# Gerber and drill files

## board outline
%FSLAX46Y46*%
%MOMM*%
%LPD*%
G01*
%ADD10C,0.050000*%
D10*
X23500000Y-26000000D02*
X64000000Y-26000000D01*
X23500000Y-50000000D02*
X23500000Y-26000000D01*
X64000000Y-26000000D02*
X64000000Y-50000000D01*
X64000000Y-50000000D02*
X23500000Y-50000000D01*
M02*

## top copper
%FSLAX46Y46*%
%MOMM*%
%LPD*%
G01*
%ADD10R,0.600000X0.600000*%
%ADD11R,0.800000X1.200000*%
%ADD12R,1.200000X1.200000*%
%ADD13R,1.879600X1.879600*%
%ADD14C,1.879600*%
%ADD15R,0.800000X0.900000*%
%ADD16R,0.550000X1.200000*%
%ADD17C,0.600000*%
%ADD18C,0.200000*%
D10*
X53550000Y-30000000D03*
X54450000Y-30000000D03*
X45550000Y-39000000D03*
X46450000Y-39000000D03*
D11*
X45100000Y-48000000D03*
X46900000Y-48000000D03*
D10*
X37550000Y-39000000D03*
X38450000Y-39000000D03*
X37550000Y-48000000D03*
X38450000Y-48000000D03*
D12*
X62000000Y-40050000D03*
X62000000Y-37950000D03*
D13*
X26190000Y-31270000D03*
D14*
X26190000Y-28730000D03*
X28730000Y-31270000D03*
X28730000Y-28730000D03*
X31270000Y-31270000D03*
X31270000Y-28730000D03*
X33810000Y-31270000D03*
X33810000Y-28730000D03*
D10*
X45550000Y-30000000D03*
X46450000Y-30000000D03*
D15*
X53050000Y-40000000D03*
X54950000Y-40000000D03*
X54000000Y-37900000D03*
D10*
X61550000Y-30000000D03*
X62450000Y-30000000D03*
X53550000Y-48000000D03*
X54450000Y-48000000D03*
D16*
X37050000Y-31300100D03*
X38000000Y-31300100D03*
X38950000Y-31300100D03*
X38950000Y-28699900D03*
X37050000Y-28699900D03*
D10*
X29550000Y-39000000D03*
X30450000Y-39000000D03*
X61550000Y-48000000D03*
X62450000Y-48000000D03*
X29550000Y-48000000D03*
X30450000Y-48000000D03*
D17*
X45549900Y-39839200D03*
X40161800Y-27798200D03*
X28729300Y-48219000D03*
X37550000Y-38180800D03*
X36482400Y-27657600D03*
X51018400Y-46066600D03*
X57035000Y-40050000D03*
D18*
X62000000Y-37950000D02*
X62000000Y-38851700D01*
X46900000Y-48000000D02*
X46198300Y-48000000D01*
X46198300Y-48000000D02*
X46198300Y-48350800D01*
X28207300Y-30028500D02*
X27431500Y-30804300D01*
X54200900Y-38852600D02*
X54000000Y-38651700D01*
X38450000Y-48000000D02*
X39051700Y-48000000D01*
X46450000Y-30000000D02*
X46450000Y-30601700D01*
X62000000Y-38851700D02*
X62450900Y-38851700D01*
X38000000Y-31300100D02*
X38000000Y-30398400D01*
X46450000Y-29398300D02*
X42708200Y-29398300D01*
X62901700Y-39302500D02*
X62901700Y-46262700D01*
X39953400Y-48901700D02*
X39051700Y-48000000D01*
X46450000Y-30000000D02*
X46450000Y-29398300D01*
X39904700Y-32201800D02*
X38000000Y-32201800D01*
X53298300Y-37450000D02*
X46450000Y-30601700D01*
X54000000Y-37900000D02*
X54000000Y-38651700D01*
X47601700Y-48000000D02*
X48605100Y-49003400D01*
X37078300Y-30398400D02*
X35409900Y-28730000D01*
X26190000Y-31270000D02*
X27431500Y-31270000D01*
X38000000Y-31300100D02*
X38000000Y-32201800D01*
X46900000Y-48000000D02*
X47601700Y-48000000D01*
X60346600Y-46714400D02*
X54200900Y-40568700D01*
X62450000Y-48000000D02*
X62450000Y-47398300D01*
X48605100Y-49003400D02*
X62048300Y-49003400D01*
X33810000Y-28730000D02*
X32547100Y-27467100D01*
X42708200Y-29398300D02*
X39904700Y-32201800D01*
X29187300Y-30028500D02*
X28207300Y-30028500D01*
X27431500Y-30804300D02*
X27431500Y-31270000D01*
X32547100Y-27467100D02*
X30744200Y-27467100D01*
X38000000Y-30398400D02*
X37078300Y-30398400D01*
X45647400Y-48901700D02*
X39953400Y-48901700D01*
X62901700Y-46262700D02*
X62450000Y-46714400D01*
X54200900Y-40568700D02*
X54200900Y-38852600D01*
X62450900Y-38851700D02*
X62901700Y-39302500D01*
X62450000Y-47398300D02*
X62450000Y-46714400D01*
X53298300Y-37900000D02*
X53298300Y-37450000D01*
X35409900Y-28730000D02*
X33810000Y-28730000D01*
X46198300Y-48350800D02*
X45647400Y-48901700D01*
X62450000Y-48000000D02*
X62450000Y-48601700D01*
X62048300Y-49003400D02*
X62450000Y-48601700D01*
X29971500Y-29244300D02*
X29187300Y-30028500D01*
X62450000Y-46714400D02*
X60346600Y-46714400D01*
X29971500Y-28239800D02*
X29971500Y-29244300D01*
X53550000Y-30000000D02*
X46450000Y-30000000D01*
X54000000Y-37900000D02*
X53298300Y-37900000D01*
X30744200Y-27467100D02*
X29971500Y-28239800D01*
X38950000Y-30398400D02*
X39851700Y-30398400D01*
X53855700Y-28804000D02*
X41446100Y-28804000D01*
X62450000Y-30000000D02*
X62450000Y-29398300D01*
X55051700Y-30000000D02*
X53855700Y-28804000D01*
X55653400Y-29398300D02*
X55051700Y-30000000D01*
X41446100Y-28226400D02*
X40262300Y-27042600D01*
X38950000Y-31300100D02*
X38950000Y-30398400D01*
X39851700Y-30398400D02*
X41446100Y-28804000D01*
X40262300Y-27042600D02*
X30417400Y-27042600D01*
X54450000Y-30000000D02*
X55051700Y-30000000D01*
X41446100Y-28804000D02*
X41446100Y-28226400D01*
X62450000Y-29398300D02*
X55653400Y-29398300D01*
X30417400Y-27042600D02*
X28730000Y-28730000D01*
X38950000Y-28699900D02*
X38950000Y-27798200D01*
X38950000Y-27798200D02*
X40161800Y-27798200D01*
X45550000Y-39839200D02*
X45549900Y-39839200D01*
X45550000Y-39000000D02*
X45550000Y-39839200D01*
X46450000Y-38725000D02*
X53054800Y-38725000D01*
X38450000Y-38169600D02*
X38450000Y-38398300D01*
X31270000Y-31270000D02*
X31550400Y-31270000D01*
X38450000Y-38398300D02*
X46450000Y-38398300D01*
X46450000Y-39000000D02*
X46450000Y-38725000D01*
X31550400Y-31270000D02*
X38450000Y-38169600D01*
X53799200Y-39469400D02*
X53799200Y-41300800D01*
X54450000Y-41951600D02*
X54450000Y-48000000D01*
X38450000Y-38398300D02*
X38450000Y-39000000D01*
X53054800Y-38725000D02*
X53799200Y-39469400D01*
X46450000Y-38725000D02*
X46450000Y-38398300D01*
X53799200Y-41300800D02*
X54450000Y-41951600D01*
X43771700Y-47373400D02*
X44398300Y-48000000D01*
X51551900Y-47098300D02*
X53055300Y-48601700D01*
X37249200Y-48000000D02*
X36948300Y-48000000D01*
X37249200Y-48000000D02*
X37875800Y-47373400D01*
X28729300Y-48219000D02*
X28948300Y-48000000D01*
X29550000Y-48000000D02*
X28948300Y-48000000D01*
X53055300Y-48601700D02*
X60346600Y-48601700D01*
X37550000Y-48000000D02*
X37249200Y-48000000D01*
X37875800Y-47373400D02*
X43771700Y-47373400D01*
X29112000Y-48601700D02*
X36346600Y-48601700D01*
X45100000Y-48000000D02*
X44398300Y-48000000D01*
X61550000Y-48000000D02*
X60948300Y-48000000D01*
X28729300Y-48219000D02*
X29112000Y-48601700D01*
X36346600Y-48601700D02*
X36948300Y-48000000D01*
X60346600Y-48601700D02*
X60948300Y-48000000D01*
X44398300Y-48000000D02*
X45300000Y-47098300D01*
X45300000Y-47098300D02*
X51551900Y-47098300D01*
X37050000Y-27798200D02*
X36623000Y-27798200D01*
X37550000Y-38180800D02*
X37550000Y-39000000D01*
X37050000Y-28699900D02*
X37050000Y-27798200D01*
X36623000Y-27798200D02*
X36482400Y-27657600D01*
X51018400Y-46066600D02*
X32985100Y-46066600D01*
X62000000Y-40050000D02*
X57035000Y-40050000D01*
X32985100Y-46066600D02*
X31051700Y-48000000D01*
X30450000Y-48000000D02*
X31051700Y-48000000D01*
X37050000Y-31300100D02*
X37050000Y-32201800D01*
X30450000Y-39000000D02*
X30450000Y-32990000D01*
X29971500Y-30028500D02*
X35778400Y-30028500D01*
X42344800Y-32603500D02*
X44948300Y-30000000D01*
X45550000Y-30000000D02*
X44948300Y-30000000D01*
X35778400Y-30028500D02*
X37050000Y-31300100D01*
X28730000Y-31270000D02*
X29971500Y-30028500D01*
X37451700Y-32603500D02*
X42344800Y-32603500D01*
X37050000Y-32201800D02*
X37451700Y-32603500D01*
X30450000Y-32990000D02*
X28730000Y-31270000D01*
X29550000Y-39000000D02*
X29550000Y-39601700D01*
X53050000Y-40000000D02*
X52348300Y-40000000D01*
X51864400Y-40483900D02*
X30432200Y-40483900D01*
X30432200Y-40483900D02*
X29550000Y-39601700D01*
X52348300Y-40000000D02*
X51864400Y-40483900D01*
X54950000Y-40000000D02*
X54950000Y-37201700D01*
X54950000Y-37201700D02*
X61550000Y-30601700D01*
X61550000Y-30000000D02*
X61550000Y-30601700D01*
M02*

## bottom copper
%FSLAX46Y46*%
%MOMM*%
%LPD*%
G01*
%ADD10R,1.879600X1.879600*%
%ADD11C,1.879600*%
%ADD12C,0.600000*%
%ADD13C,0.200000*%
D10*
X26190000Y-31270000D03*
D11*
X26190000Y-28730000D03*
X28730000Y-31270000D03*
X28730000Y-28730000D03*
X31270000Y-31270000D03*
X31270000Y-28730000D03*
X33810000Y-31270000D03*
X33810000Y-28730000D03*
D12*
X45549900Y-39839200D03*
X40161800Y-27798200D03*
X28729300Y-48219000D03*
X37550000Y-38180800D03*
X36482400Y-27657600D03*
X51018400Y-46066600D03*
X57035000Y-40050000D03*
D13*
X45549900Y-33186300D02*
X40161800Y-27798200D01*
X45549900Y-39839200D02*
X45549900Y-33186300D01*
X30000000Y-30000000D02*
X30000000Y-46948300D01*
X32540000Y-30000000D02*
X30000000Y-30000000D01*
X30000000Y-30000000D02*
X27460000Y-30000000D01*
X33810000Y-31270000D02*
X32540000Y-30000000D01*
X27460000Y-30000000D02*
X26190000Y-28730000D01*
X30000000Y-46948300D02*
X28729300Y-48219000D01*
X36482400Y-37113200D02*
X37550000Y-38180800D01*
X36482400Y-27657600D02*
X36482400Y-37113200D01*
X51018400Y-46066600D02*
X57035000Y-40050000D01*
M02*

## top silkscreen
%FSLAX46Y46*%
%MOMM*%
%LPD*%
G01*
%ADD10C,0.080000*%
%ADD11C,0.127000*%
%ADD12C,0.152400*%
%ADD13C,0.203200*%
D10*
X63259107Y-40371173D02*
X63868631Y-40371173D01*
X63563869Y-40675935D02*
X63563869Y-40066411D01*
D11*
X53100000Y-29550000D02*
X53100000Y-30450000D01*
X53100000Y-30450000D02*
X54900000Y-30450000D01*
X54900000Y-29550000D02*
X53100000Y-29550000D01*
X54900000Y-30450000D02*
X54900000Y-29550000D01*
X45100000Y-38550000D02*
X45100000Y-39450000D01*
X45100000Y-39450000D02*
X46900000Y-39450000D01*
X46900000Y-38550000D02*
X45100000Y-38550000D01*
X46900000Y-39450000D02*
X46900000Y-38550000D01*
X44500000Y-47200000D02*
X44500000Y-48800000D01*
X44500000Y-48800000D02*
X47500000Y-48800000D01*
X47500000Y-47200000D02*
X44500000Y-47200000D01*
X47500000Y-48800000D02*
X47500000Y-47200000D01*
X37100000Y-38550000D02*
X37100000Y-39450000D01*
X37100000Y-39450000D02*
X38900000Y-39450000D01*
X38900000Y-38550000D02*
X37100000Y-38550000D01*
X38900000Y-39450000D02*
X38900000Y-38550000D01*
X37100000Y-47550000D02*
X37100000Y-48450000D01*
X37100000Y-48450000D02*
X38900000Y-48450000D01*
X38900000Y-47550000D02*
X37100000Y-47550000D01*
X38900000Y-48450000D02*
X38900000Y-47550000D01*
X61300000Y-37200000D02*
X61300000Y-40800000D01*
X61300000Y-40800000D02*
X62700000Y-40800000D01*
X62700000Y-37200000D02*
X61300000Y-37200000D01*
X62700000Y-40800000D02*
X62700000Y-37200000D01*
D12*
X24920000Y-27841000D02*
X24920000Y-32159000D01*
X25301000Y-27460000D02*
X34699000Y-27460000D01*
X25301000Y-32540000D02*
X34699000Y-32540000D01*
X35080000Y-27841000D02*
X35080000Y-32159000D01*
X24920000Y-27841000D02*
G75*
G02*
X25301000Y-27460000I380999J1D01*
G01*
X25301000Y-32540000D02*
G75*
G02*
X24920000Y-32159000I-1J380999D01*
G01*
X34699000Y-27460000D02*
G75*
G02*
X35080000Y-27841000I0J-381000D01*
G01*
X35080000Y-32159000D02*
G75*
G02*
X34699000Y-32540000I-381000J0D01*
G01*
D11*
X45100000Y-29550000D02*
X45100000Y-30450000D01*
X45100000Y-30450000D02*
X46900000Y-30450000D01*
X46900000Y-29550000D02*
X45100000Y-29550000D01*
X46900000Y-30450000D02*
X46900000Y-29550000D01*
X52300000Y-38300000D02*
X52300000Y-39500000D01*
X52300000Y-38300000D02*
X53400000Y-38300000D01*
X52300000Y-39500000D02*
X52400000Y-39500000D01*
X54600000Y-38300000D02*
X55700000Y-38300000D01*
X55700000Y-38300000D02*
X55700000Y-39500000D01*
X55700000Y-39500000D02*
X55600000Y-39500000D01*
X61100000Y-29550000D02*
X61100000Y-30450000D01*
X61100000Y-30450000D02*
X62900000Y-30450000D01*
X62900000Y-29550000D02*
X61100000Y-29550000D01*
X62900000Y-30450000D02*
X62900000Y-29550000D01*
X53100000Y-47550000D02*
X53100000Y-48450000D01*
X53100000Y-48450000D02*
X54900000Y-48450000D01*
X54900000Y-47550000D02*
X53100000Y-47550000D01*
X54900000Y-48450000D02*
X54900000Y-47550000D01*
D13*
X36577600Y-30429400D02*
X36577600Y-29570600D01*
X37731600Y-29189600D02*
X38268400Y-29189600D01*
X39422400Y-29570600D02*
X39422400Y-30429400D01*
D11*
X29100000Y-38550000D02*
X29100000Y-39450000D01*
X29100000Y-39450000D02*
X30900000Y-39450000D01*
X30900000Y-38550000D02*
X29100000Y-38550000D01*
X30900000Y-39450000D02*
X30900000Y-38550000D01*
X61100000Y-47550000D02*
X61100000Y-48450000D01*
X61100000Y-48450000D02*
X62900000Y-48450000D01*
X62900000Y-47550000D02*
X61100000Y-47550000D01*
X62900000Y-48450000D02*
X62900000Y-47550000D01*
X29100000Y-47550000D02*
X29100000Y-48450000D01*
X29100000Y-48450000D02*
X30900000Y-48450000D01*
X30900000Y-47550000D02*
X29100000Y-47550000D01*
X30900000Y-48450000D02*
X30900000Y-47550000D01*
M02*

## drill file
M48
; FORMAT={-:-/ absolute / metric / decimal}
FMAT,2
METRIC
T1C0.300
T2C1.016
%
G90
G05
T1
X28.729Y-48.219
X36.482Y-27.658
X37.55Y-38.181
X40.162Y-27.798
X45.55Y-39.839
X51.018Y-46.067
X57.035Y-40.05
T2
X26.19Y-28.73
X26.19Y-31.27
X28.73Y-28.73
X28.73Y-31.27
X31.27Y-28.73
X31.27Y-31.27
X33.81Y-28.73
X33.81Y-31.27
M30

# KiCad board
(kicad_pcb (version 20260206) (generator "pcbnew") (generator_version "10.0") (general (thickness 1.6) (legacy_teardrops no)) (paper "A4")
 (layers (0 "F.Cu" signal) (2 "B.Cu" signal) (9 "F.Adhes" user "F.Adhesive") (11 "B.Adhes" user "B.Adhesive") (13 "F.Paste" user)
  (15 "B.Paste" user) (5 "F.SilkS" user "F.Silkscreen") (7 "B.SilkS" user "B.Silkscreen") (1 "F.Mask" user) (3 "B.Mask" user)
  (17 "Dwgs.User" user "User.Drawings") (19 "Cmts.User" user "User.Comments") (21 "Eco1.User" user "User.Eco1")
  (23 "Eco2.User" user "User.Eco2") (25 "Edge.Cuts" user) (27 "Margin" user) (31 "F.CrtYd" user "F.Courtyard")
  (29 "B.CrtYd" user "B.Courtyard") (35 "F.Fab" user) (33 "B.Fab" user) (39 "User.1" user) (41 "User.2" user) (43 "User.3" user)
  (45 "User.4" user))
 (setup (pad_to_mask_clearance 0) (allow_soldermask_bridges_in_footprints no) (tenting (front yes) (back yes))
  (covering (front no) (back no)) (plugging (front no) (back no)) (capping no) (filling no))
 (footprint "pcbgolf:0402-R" (layer "F.Cu") (at 54 30)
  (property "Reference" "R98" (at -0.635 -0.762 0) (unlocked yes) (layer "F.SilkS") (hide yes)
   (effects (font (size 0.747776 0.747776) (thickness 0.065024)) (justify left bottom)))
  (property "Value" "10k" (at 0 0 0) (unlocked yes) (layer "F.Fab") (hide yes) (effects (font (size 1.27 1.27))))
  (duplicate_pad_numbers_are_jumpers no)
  (fp_line (start -0.9 -0.45) (end -0.9 0.45) (stroke (width 0.127) (type solid)) (layer "F.SilkS"))
  (fp_line (start -0.9 0.45) (end 0.9 0.45) (stroke (width 0.127) (type solid)) (layer "F.SilkS"))
  (fp_line (start 0.9 -0.45) (end -0.9 -0.45) (stroke (width 0.127) (type solid)) (layer "F.SilkS"))
  (fp_line (start 0.9 0.45) (end 0.9 -0.45) (stroke (width 0.127) (type solid)) (layer "F.SilkS"))
  (pad "1" smd rect (at -0.45 0) (size 0.6 0.6) (layers "F.Cu" "F.Mask" "F.Paste") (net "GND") (solder_mask_margin 0.0508)
   (solder_paste_margin 0) (thermal_bridge_angle 0))
  (pad "2" smd rect (at 0.45 0) (size 0.6 0.6) (layers "F.Cu" "F.Mask" "F.Paste") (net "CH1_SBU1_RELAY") (solder_mask_margin 0.0508)
   (solder_paste_margin 0) (thermal_bridge_angle 0)))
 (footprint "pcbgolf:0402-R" (layer "F.Cu") (at 46 39)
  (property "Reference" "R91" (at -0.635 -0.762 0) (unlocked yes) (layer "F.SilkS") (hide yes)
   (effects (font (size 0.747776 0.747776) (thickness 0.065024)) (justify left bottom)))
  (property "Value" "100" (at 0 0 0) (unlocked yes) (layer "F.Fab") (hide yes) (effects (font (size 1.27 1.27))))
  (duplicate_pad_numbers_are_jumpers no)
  (fp_line (start -0.9 -0.45) (end -0.9 0.45) (stroke (width 0.127) (type solid)) (layer "F.SilkS"))
  (fp_line (start -0.9 0.45) (end 0.9 0.45) (stroke (width 0.127) (type solid)) (layer "F.SilkS"))
  (fp_line (start 0.9 -0.45) (end -0.9 -0.45) (stroke (width 0.127) (type solid)) (layer "F.SilkS"))
  (fp_line (start 0.9 0.45) (end 0.9 -0.45) (stroke (width 0.127) (type solid)) (layer "F.SilkS"))
  (pad "1" smd rect (at -0.45 0) (size 0.6 0.6) (layers "F.Cu" "F.Mask" "F.Paste") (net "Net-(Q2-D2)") (solder_mask_margin 0.0508)
   (solder_paste_margin 0) (thermal_bridge_angle 0))
  (pad "2" smd rect (at 0.45 0) (size 0.6 0.6) (layers "F.Cu" "F.Mask" "F.Paste") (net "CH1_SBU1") (solder_mask_margin 0.0508)
   (solder_paste_margin 0) (thermal_bridge_angle 0)))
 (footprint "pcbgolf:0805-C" (layer "F.Cu") (at 46 48)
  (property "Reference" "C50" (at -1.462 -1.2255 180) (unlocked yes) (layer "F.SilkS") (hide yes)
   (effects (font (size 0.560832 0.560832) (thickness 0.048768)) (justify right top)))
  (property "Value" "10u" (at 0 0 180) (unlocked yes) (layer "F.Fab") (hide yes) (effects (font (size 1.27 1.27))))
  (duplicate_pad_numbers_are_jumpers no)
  (fp_line (start -1.5 -0.8) (end -1.5 0.8) (stroke (width 0.127) (type solid)) (layer "F.SilkS"))
  (fp_line (start -1.5 0.8) (end 1.5 0.8) (stroke (width 0.127) (type solid)) (layer "F.SilkS"))
  (fp_line (start 1.5 -0.8) (end -1.5 -0.8) (stroke (width 0.127) (type solid)) (layer "F.SilkS"))
  (fp_line (start 1.5 0.8) (end 1.5 -0.8) (stroke (width 0.127) (type solid)) (layer "F.SilkS"))
  (pad "1" smd rect (at -0.9 0) (size 0.8 1.2) (layers "F.Cu" "F.Mask" "F.Paste") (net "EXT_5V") (solder_mask_margin 0.0508)
   (solder_paste_margin 0) (thermal_bridge_angle 0))
  (pad "2" smd rect (at 0.9 0) (size 0.8 1.2) (layers "F.Cu" "F.Mask" "F.Paste") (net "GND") (solder_mask_margin 0.0508)
   (solder_paste_margin 0) (thermal_bridge_angle 0)))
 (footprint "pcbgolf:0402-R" (layer "F.Cu") (at 38 39)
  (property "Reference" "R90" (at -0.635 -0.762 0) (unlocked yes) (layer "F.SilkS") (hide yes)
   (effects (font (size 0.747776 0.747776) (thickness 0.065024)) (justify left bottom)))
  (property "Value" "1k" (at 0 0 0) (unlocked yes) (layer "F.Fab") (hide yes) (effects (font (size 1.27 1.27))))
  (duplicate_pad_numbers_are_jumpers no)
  (fp_line (start -0.9 -0.45) (end -0.9 0.45) (stroke (width 0.127) (type solid)) (layer "F.SilkS"))
  (fp_line (start -0.9 0.45) (end 0.9 0.45) (stroke (width 0.127) (type solid)) (layer "F.SilkS"))
  (fp_line (start 0.9 -0.45) (end -0.9 -0.45) (stroke (width 0.127) (type solid)) (layer "F.SilkS"))
  (fp_line (start 0.9 0.45) (end 0.9 -0.45) (stroke (width 0.127) (type solid)) (layer "F.SilkS"))
  (pad "1" smd rect (at -0.45 0) (size 0.6 0.6) (layers "F.Cu" "F.Mask" "F.Paste") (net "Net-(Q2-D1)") (solder_mask_margin 0.0508)
   (solder_paste_margin 0) (thermal_bridge_angle 0))
  (pad "2" smd rect (at 0.45 0) (size 0.6 0.6) (layers "F.Cu" "F.Mask" "F.Paste") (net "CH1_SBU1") (solder_mask_margin 0.0508)
   (solder_paste_margin 0) (thermal_bridge_angle 0)))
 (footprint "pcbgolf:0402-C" (layer "F.Cu") (at 38 48)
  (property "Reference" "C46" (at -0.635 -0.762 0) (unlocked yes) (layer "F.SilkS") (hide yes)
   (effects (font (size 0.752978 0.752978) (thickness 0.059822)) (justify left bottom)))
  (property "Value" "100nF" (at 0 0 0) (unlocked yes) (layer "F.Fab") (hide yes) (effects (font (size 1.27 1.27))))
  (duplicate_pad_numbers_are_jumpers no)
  (fp_line (start -0.9 -0.45) (end -0.9 0.45) (stroke (width 0.127) (type solid)) (layer "F.SilkS"))
  (fp_line (start -0.9 0.45) (end 0.9 0.45) (stroke (width 0.127) (type solid)) (layer "F.SilkS"))
  (fp_line (start 0.9 -0.45) (end -0.9 -0.45) (stroke (width 0.127) (type solid)) (layer "F.SilkS"))
  (fp_line (start 0.9 0.45) (end 0.9 -0.45) (stroke (width 0.127) (type solid)) (layer "F.SilkS"))
  (pad "1" smd rect (at -0.45 0) (size 0.6 0.6) (layers "F.Cu" "F.Mask" "F.Paste") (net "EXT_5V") (solder_mask_margin 0.0508)
   (solder_paste_margin 0) (thermal_bridge_angle 0))
  (pad "2" smd rect (at 0.45 0) (size 0.6 0.6) (layers "F.Cu" "F.Mask" "F.Paste") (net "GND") (solder_mask_margin 0.0508)
   (solder_paste_margin 0) (thermal_bridge_angle 0)))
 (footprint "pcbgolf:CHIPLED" (layer "F.Cu") (at 62 39)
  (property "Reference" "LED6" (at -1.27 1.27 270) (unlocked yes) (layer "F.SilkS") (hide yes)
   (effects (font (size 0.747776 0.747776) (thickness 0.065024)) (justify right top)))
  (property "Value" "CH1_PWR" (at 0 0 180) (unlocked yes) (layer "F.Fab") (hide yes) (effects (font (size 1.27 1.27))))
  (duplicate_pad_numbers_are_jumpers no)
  (fp_line (start -0.7 -1.8) (end -0.7 1.8) (stroke (width 0.127) (type solid)) (layer "F.SilkS"))
  (fp_line (start -0.7 1.8) (end 0.7 1.8) (stroke (width 0.127) (type solid)) (layer "F.SilkS"))
  (fp_line (start 0.7 -1.8) (end -0.7 -1.8) (stroke (width 0.127) (type solid)) (layer "F.SilkS"))
  (fp_line (start 0.7 1.8) (end 0.7 -1.8) (stroke (width 0.127) (type solid)) (layer "F.SilkS"))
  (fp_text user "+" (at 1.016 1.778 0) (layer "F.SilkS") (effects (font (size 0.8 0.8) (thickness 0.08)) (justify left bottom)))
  (pad "A" smd rect (at 0 1.05) (size 1.2 1.2) (layers "F.Cu" "F.Mask" "F.Paste") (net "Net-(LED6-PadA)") (solder_mask_margin 0.0508)
   (solder_paste_margin 0) (thermal_bridge_angle 0))
  (pad "C" smd rect (at 0 -1.05) (size 1.2 1.2) (layers "F.Cu" "F.Mask" "F.Paste") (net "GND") (solder_mask_margin 0.0508)
   (solder_paste_margin 0) (thermal_bridge_angle 0)))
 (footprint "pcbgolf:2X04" (layer "F.Cu") (at 30 30)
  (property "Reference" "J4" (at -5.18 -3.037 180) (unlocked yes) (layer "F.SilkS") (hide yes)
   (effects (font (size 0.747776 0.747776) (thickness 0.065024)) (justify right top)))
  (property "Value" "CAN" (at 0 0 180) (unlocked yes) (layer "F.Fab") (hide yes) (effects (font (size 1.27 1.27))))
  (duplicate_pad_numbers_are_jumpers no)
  (fp_line (start -5.08 -2.159) (end -5.08 2.159) (stroke (width 0.1524) (type solid)) (layer "F.SilkS"))
  (fp_line (start -4.699 -2.54) (end 4.699 -2.54) (stroke (width 0.1524) (type solid)) (layer "F.SilkS"))
  (fp_line (start -4.699 2.54) (end 4.699 2.54) (stroke (width 0.1524) (type solid)) (layer "F.SilkS"))
  (fp_line (start 5.08 -2.159) (end 5.08 2.159) (stroke (width 0.1524) (type solid)) (layer "F.SilkS"))
  (fp_arc (start -5.08 -2.159) (mid -4.968408 -2.428408) (end -4.699 -2.54) (stroke (width 0.1524) (type solid)) (layer "F.SilkS"))
  (fp_arc (start -4.699 2.54) (mid -4.968408 2.428408) (end -5.08 2.159) (stroke (width 0.1524) (type solid)) (layer "F.SilkS"))
  (fp_arc (start 4.699 -2.54) (mid 4.968408 -2.428408) (end 5.08 -2.159) (stroke (width 0.1524) (type solid)) (layer "F.SilkS"))
  (fp_arc (start 5.08 2.159) (mid 4.968408 2.428408) (end 4.699 2.54) (stroke (width 0.1524) (type solid)) (layer "F.SilkS"))
  (pad "1" thru_hole rect (at -3.81 1.27 90) (size 1.8796 1.8796) (drill 1.016) (layers "*.Cu" "*.Mask") (remove_unused_layers no)
   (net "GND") (solder_mask_margin 0.0508) (thermal_bridge_angle 0))
  (pad "2" thru_hole circle (at -3.81 -1.27 90) (size 1.8796 1.8796) (drill 1.016) (layers "*.Cu" "*.Mask") (remove_unused_layers no)
   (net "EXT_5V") (solder_mask_margin 0.0508) (thermal_bridge_angle 0))
  (pad "3" thru_hole circle (at -1.27 1.27 90) (size 1.8796 1.8796) (drill 1.016) (layers "*.Cu" "*.Mask") (remove_unused_layers no)
   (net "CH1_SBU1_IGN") (solder_mask_margin 0.0508) (thermal_bridge_angle 0))
  (pad "4" thru_hole circle (at -1.27 -1.27 90) (size 1.8796 1.8796) (drill 1.016) (layers "*.Cu" "*.Mask") (remove_unused_layers no)
   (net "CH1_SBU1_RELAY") (solder_mask_margin 0.0508) (thermal_bridge_angle 0))
  (pad "5" thru_hole circle (at 1.27 1.27 90) (size 1.8796 1.8796) (drill 1.016) (layers "*.Cu" "*.Mask") (remove_unused_layers no)
   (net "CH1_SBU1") (solder_mask_margin 0.0508) (thermal_bridge_angle 0))
  (pad "6" thru_hole circle (at 1.27 -1.27 90) (size 1.8796 1.8796) (drill 1.016) (layers "*.Cu" "*.Mask") (remove_unused_layers no)
   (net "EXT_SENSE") (solder_mask_margin 0.0508) (thermal_bridge_angle 0))
  (pad "7" thru_hole circle (at 3.81 1.27 90) (size 1.8796 1.8796) (drill 1.016) (layers "*.Cu" "*.Mask") (remove_unused_layers no)
   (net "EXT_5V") (solder_mask_margin 0.0508) (thermal_bridge_angle 0))
  (pad "8" thru_hole circle (at 3.81 -1.27 90) (size 1.8796 1.8796) (drill 1.016) (layers "*.Cu" "*.Mask") (remove_unused_layers no)
   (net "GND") (solder_mask_margin 0.0508) (thermal_bridge_angle 0)))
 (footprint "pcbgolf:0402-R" (layer "F.Cu") (at 46 30)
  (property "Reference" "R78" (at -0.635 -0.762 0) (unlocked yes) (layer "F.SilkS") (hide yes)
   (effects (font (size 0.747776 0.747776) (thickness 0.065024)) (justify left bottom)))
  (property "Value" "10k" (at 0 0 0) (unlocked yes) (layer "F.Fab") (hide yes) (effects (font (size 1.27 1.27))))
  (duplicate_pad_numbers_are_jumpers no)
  (fp_line (start -0.9 -0.45) (end -0.9 0.45) (stroke (width 0.127) (type solid)) (layer "F.SilkS"))
  (fp_line (start -0.9 0.45) (end 0.9 0.45) (stroke (width 0.127) (type solid)) (layer "F.SilkS"))
  (fp_line (start 0.9 -0.45) (end -0.9 -0.45) (stroke (width 0.127) (type solid)) (layer "F.SilkS"))
  (fp_line (start 0.9 0.45) (end 0.9 -0.45) (stroke (width 0.127) (type solid)) (layer "F.SilkS"))
  (pad "1" smd rect (at -0.45 0) (size 0.6 0.6) (layers "F.Cu" "F.Mask" "F.Paste") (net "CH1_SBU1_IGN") (solder_mask_margin 0.0508)
   (solder_paste_margin 0) (thermal_bridge_angle 0))
  (pad "2" smd rect (at 0.45 0) (size 0.6 0.6) (layers "F.Cu" "F.Mask" "F.Paste") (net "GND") (solder_mask_margin 0.0508)
   (solder_paste_margin 0) (thermal_bridge_angle 0)))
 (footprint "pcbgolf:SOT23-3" (layer "F.Cu") (at 54 39)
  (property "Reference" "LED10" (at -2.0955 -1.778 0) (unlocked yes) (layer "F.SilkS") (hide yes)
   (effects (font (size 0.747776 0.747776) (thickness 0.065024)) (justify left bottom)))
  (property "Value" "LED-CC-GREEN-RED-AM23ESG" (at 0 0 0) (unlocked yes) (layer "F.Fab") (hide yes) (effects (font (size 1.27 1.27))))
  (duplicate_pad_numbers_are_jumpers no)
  (fp_line (start -1.7 -0.7) (end -1.7 0.5) (stroke (width 0.127) (type solid)) (layer "F.SilkS"))
  (fp_line (start -1.7 -0.7) (end -0.6 -0.7) (stroke (width 0.127) (type solid)) (layer "F.SilkS"))
  (fp_line (start -1.7 0.5) (end -1.6 0.5) (stroke (width 0.127) (type solid)) (layer "F.SilkS"))
  (fp_line (start 0.6 -0.7) (end 1.7 -0.7) (stroke (width 0.127) (type solid)) (layer "F.SilkS"))
  (fp_line (start 1.7 -0.7) (end 1.7 0.5) (stroke (width 0.127) (type solid)) (layer "F.SilkS"))
  (fp_line (start 1.7 0.5) (end 1.6 0.5) (stroke (width 0.127) (type solid)) (layer "F.SilkS"))
  (pad "1" smd rect (at -0.95 1) (size 0.8 0.9) (layers "F.Cu" "F.Mask" "F.Paste") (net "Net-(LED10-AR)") (solder_mask_margin 0.0508)
   (solder_paste_margin 0) (thermal_bridge_angle 0))
  (pad "2" smd rect (at 0.95 1) (size 0.8 0.9) (layers "F.Cu" "F.Mask" "F.Paste") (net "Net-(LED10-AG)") (solder_mask_margin 0.0508)
   (solder_paste_margin 0) (thermal_bridge_angle 0))
  (pad "3" smd rect (at 0 -1.1) (size 0.8 0.9) (layers "F.Cu" "F.Mask" "F.Paste") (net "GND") (solder_mask_margin 0.0508)
   (solder_paste_margin 0) (thermal_bridge_angle 0)))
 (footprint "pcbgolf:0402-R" (layer "F.Cu") (at 62 30)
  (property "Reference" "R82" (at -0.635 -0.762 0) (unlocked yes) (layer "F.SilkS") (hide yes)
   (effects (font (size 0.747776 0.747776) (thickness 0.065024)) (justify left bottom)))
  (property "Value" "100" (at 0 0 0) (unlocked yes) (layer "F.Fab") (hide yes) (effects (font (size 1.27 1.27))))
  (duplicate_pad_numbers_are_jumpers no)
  (fp_line (start -0.9 -0.45) (end -0.9 0.45) (stroke (width 0.127) (type solid)) (layer "F.SilkS"))
  (fp_line (start -0.9 0.45) (end 0.9 0.45) (stroke (width 0.127) (type solid)) (layer "F.SilkS"))
  (fp_line (start 0.9 -0.45) (end -0.9 -0.45) (stroke (width 0.127) (type solid)) (layer "F.SilkS"))
  (fp_line (start 0.9 0.45) (end 0.9 -0.45) (stroke (width 0.127) (type solid)) (layer "F.SilkS"))
  (pad "1" smd rect (at -0.45 0) (size 0.6 0.6) (layers "F.Cu" "F.Mask" "F.Paste") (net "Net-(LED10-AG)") (solder_mask_margin 0.0508)
   (solder_paste_margin 0) (thermal_bridge_angle 0))
  (pad "2" smd rect (at 0.45 0) (size 0.6 0.6) (layers "F.Cu" "F.Mask" "F.Paste") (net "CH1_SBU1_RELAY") (solder_mask_margin 0.0508)
   (solder_paste_margin 0) (thermal_bridge_angle 0)))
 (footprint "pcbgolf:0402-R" (layer "F.Cu") (at 54 48)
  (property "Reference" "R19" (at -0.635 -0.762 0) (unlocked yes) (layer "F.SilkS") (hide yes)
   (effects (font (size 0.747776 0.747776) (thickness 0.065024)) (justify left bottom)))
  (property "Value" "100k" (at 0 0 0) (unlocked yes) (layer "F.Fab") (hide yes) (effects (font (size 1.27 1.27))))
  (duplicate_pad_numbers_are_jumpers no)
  (fp_line (start -0.9 -0.45) (end -0.9 0.45) (stroke (width 0.127) (type solid)) (layer "F.SilkS"))
  (fp_line (start -0.9 0.45) (end 0.9 0.45) (stroke (width 0.127) (type solid)) (layer "F.SilkS"))
  (fp_line (start 0.9 -0.45) (end -0.9 -0.45) (stroke (width 0.127) (type solid)) (layer "F.SilkS"))
  (fp_line (start 0.9 0.45) (end 0.9 -0.45) (stroke (width 0.127) (type solid)) (layer "F.SilkS"))
  (pad "1" smd rect (at -0.45 0) (size 0.6 0.6) (layers "F.Cu" "F.Mask" "F.Paste") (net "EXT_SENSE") (solder_mask_margin 0.0508)
   (solder_paste_margin 0) (thermal_bridge_angle 0))
  (pad "2" smd rect (at 0.45 0) (size 0.6 0.6) (layers "F.Cu" "F.Mask" "F.Paste") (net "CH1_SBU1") (solder_mask_margin 0.0508)
   (solder_paste_margin 0) (thermal_bridge_angle 0)))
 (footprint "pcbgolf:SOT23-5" (layer "F.Cu") (at 38 30)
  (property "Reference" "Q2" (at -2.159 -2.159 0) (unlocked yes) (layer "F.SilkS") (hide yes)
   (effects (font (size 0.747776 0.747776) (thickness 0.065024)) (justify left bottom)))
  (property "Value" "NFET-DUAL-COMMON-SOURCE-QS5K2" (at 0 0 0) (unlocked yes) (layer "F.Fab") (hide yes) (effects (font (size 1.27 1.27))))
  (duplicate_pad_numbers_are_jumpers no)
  (fp_line (start -1.4224 0.4294) (end -1.4224 -0.4294) (stroke (width 0.2032) (type solid)) (layer "F.SilkS"))
  (fp_line (start -0.2684 -0.8104) (end 0.2684 -0.8104) (stroke (width 0.2032) (type solid)) (layer "F.SilkS"))
  (fp_line (start 1.4224 -0.4294) (end 1.4224 0.4294) (stroke (width 0.2032) (type solid)) (layer "F.SilkS"))
  (pad "1" smd rect (at -0.95 1.3001) (size 0.55 1.2) (layers "F.Cu" "F.Mask" "F.Paste") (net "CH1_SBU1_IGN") (solder_mask_margin 0.0508)
   (solder_paste_margin 0) (thermal_bridge_angle 0))
  (pad "2" smd rect (at 0 1.3001) (size 0.55 1.2) (layers "F.Cu" "F.Mask" "F.Paste") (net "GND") (solder_mask_margin 0.0508)
   (solder_paste_margin 0) (thermal_bridge_angle 0))
  (pad "3" smd rect (at 0.95 1.3001) (size 0.55 1.2) (layers "F.Cu" "F.Mask" "F.Paste") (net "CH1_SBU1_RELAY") (solder_mask_margin 0.0508)
   (solder_paste_margin 0) (thermal_bridge_angle 0))
  (pad "4" smd rect (at 0.95 -1.3001) (size 0.55 1.2) (layers "F.Cu" "F.Mask" "F.Paste") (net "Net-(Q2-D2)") (solder_mask_margin 0.0508)
   (solder_paste_margin 0) (thermal_bridge_angle 0))
  (pad "5" smd rect (at -0.95 -1.3001) (size 0.55 1.2) (layers "F.Cu" "F.Mask" "F.Paste") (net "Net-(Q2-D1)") (solder_mask_margin 0.0508)
   (solder_paste_margin 0) (thermal_bridge_angle 0)))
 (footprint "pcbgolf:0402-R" (layer "F.Cu") (at 30 39)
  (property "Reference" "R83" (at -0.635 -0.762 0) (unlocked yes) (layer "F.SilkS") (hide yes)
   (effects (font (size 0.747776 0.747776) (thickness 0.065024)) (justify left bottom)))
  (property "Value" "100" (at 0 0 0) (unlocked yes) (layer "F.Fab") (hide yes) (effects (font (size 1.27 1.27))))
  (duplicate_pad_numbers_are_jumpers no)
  (fp_line (start -0.9 -0.45) (end -0.9 0.45) (stroke (width 0.127) (type solid)) (layer "F.SilkS"))
  (fp_line (start -0.9 0.45) (end 0.9 0.45) (stroke (width 0.127) (type solid)) (layer "F.SilkS"))
  (fp_line (start 0.9 -0.45) (end -0.9 -0.45) (stroke (width 0.127) (type solid)) (layer "F.SilkS"))
  (fp_line (start 0.9 0.45) (end 0.9 -0.45) (stroke (width 0.127) (type solid)) (layer "F.SilkS"))
  (pad "1" smd rect (at -0.45 0) (size 0.6 0.6) (layers "F.Cu" "F.Mask" "F.Paste") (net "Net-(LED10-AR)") (solder_mask_margin 0.0508)
   (solder_paste_margin 0) (thermal_bridge_angle 0))
  (pad "2" smd rect (at 0.45 0) (size 0.6 0.6) (layers "F.Cu" "F.Mask" "F.Paste") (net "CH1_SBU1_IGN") (solder_mask_margin 0.0508)
   (solder_paste_margin 0) (thermal_bridge_angle 0)))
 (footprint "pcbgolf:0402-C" (layer "F.Cu") (at 62 48)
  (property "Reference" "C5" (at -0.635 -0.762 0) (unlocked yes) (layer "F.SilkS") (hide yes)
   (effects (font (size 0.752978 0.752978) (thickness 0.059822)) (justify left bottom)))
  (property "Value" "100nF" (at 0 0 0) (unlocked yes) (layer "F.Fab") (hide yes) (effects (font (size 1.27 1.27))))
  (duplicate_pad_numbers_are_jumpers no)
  (fp_line (start -0.9 -0.45) (end -0.9 0.45) (stroke (width 0.127) (type solid)) (layer "F.SilkS"))
  (fp_line (start -0.9 0.45) (end 0.9 0.45) (stroke (width 0.127) (type solid)) (layer "F.SilkS"))
  (fp_line (start 0.9 -0.45) (end -0.9 -0.45) (stroke (width 0.127) (type solid)) (layer "F.SilkS"))
  (fp_line (start 0.9 0.45) (end 0.9 -0.45) (stroke (width 0.127) (type solid)) (layer "F.SilkS"))
  (pad "1" smd rect (at -0.45 0) (size 0.6 0.6) (layers "F.Cu" "F.Mask" "F.Paste") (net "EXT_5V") (solder_mask_margin 0.0508)
   (solder_paste_margin 0) (thermal_bridge_angle 0))
  (pad "2" smd rect (at 0.45 0) (size 0.6 0.6) (layers "F.Cu" "F.Mask" "F.Paste") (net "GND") (solder_mask_margin 0.0508)
   (solder_paste_margin 0) (thermal_bridge_angle 0)))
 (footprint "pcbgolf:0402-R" (layer "F.Cu") (at 30 48)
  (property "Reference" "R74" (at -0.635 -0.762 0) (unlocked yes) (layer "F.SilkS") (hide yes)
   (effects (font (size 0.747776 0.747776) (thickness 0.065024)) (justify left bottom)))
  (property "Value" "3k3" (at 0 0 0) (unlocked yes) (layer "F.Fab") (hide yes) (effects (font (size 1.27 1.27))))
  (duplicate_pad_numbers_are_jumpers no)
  (fp_line (start -0.9 -0.45) (end -0.9 0.45) (stroke (width 0.127) (type solid)) (layer "F.SilkS"))
  (fp_line (start -0.9 0.45) (end 0.9 0.45) (stroke (width 0.127) (type solid)) (layer "F.SilkS"))
  (fp_line (start 0.9 -0.45) (end -0.9 -0.45) (stroke (width 0.127) (type solid)) (layer "F.SilkS"))
  (fp_line (start 0.9 0.45) (end 0.9 -0.45) (stroke (width 0.127) (type solid)) (layer "F.SilkS"))
  (pad "1" smd rect (at -0.45 0) (size 0.6 0.6) (layers "F.Cu" "F.Mask" "F.Paste") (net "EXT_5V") (solder_mask_margin 0.0508)
   (solder_paste_margin 0) (thermal_bridge_angle 0))
  (pad "2" smd rect (at 0.45 0) (size 0.6 0.6) (layers "F.Cu" "F.Mask" "F.Paste") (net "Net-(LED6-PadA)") (solder_mask_margin 0.0508)
   (solder_paste_margin 0) (thermal_bridge_angle 0)))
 (gr_line (start 23.5 26) (end 64 26) (stroke (width 0.05) (type default)) (layer "Edge.Cuts"))
 (gr_line (start 23.5 50) (end 23.5 26) (stroke (width 0.05) (type default)) (layer "Edge.Cuts"))
 (gr_line (start 64 26) (end 64 50) (stroke (width 0.05) (type default)) (layer "Edge.Cuts"))
 (gr_line (start 64 50) (end 23.5 50) (stroke (width 0.05) (type default)) (layer "Edge.Cuts"))
 (segment (start 62 37.95) (end 62 38.8517) (width 0.2) (layer "F.Cu") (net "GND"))
 (segment (start 46.9 48) (end 46.1983 48) (width 0.2) (layer "F.Cu") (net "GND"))
 (segment (start 46.1983 48) (end 46.1983 48.3508) (width 0.2) (layer "F.Cu") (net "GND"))
 (segment (start 28.2073 30.0285) (end 27.4315 30.8043) (width 0.2) (layer "F.Cu") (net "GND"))
 (segment (start 54.2009 38.8526) (end 54 38.6517) (width 0.2) (layer "F.Cu") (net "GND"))
 (segment (start 38.45 48) (end 39.0517 48) (width 0.2) (layer "F.Cu") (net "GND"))
 (segment (start 46.45 30) (end 46.45 30.6017) (width 0.2) (layer "F.Cu") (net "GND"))
 (segment (start 62 38.8517) (end 62.4509 38.8517) (width 0.2) (layer "F.Cu") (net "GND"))
 (segment (start 38 31.3001) (end 38 30.3984) (width 0.2) (layer "F.Cu") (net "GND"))
 (segment (start 46.45 29.3983) (end 42.7082 29.3983) (width 0.2) (layer "F.Cu") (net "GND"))
 (segment (start 62.9017 39.3025) (end 62.9017 46.2627) (width 0.2) (layer "F.Cu") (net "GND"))
 (segment (start 39.9534 48.9017) (end 39.0517 48) (width 0.2) (layer "F.Cu") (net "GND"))
 (segment (start 46.45 30) (end 46.45 29.3983) (width 0.2) (layer "F.Cu") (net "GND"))
 (segment (start 39.9047 32.2018) (end 38 32.2018) (width 0.2) (layer "F.Cu") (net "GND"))
 (segment (start 53.2983 37.45) (end 46.45 30.6017) (width 0.2) (layer "F.Cu") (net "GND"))
 (segment (start 54 37.9) (end 54 38.6517) (width 0.2) (layer "F.Cu") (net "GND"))
 (segment (start 47.6017 48) (end 48.6051 49.0034) (width 0.2) (layer "F.Cu") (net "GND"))
 (segment (start 37.0783 30.3984) (end 35.4099 28.73) (width 0.2) (layer "F.Cu") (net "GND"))
 (segment (start 26.19 31.27) (end 27.4315 31.27) (width 0.2) (layer "F.Cu") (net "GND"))
 (segment (start 38 31.3001) (end 38 32.2018) (width 0.2) (layer "F.Cu") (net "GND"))
 (segment (start 46.9 48) (end 47.6017 48) (width 0.2) (layer "F.Cu") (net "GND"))
 (segment (start 60.3466 46.7144) (end 54.2009 40.5687) (width 0.2) (layer "F.Cu") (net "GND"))
 (segment (start 62.45 48) (end 62.45 47.3983) (width 0.2) (layer "F.Cu") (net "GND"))
 (segment (start 48.6051 49.0034) (end 62.0483 49.0034) (width 0.2) (layer "F.Cu") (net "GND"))
 (segment (start 33.81 28.73) (end 32.5471 27.4671) (width 0.2) (layer "F.Cu") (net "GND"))
 (segment (start 42.7082 29.3983) (end 39.9047 32.2018) (width 0.2) (layer "F.Cu") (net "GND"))
 (segment (start 29.1873 30.0285) (end 28.2073 30.0285) (width 0.2) (layer "F.Cu") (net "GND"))
 (segment (start 27.4315 30.8043) (end 27.4315 31.27) (width 0.2) (layer "F.Cu") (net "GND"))
 (segment (start 32.5471 27.4671) (end 30.7442 27.4671) (width 0.2) (layer "F.Cu") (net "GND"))
 (segment (start 38 30.3984) (end 37.0783 30.3984) (width 0.2) (layer "F.Cu") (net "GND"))
 (segment (start 45.6474 48.9017) (end 39.9534 48.9017) (width 0.2) (layer "F.Cu") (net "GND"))
 (segment (start 62.9017 46.2627) (end 62.45 46.7144) (width 0.2) (layer "F.Cu") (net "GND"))
 (segment (start 54.2009 40.5687) (end 54.2009 38.8526) (width 0.2) (layer "F.Cu") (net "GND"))
 (segment (start 62.4509 38.8517) (end 62.9017 39.3025) (width 0.2) (layer "F.Cu") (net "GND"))
 (segment (start 62.45 47.3983) (end 62.45 46.7144) (width 0.2) (layer "F.Cu") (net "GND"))
 (segment (start 53.2983 37.9) (end 53.2983 37.45) (width 0.2) (layer "F.Cu") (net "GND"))
 (segment (start 35.4099 28.73) (end 33.81 28.73) (width 0.2) (layer "F.Cu") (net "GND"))
 (segment (start 46.1983 48.3508) (end 45.6474 48.9017) (width 0.2) (layer "F.Cu") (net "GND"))
 (segment (start 62.45 48) (end 62.45 48.6017) (width 0.2) (layer "F.Cu") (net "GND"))
 (segment (start 62.0483 49.0034) (end 62.45 48.6017) (width 0.2) (layer "F.Cu") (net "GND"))
 (segment (start 29.9715 29.2443) (end 29.1873 30.0285) (width 0.2) (layer "F.Cu") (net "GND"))
 (segment (start 62.45 46.7144) (end 60.3466 46.7144) (width 0.2) (layer "F.Cu") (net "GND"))
 (segment (start 29.9715 28.2398) (end 29.9715 29.2443) (width 0.2) (layer "F.Cu") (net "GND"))
 (segment (start 53.55 30) (end 46.45 30) (width 0.2) (layer "F.Cu") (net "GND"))
 (segment (start 54 37.9) (end 53.2983 37.9) (width 0.2) (layer "F.Cu") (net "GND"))
 (segment (start 30.7442 27.4671) (end 29.9715 28.2398) (width 0.2) (layer "F.Cu") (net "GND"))
 (segment (start 38.95 30.3984) (end 39.8517 30.3984) (width 0.2) (layer "F.Cu") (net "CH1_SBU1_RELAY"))
 (segment (start 53.8557 28.804) (end 41.4461 28.804) (width 0.2) (layer "F.Cu") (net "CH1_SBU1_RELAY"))
 (segment (start 62.45 30) (end 62.45 29.3983) (width 0.2) (layer "F.Cu") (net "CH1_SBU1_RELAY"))
 (segment (start 55.0517 30) (end 53.8557 28.804) (width 0.2) (layer "F.Cu") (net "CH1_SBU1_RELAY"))
 (segment (start 55.6534 29.3983) (end 55.0517 30) (width 0.2) (layer "F.Cu") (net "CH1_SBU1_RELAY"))
 (segment (start 41.4461 28.2264) (end 40.2623 27.0426) (width 0.2) (layer "F.Cu") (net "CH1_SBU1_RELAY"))
 (segment (start 38.95 31.3001) (end 38.95 30.3984) (width 0.2) (layer "F.Cu") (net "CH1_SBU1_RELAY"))
 (segment (start 39.8517 30.3984) (end 41.4461 28.804) (width 0.2) (layer "F.Cu") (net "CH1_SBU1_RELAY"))
 (segment (start 40.2623 27.0426) (end 30.4174 27.0426) (width 0.2) (layer "F.Cu") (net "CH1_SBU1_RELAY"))
 (segment (start 54.45 30) (end 55.0517 30) (width 0.2) (layer "F.Cu") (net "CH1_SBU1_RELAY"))
 (segment (start 41.4461 28.804) (end 41.4461 28.2264) (width 0.2) (layer "F.Cu") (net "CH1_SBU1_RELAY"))
 (segment (start 62.45 29.3983) (end 55.6534 29.3983) (width 0.2) (layer "F.Cu") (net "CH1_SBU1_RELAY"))
 (segment (start 30.4174 27.0426) (end 28.73 28.73) (width 0.2) (layer "F.Cu") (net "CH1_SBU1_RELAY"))
 (segment (start 38.95 28.6999) (end 38.95 27.7982) (width 0.2) (layer "F.Cu") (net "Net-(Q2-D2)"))
 (segment (start 38.95 27.7982) (end 40.1618 27.7982) (width 0.2) (layer "F.Cu") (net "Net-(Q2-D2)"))
 (segment (start 45.55 39.8392) (end 45.5499 39.8392) (width 0.2) (layer "F.Cu") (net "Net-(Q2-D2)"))
 (segment (start 45.55 39) (end 45.55 39.8392) (width 0.2) (layer "F.Cu") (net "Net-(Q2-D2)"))
 (via (at 45.5499 39.8392) (size 0.6) (drill 0.3) (layers "F.Cu" "B.Cu") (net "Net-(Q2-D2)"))
 (via (at 40.1618 27.7982) (size 0.6) (drill 0.3) (layers "F.Cu" "B.Cu") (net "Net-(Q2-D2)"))
 (segment (start 45.5499 33.1863) (end 40.1618 27.7982) (width 0.2) (layer "B.Cu") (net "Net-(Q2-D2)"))
 (segment (start 45.5499 39.8392) (end 45.5499 33.1863) (width 0.2) (layer "B.Cu") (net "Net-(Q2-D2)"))
 (segment (start 46.45 38.725) (end 53.0548 38.725) (width 0.2) (layer "F.Cu") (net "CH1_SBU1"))
 (segment (start 38.45 38.1696) (end 38.45 38.3983) (width 0.2) (layer "F.Cu") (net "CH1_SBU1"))
 (segment (start 31.27 31.27) (end 31.5504 31.27) (width 0.2) (layer "F.Cu") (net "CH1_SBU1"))
 (segment (start 38.45 38.3983) (end 46.45 38.3983) (width 0.2) (layer "F.Cu") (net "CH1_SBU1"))
 (segment (start 46.45 39) (end 46.45 38.725) (width 0.2) (layer "F.Cu") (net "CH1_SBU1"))
 (segment (start 31.5504 31.27) (end 38.45 38.1696) (width 0.2) (layer "F.Cu") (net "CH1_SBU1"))
 (segment (start 53.7992 39.4694) (end 53.7992 41.3008) (width 0.2) (layer "F.Cu") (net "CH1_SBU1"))
 (segment (start 54.45 41.9516) (end 54.45 48) (width 0.2) (layer "F.Cu") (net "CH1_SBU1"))
 (segment (start 38.45 38.3983) (end 38.45 39) (width 0.2) (layer "F.Cu") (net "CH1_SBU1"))
 (segment (start 53.0548 38.725) (end 53.7992 39.4694) (width 0.2) (layer "F.Cu") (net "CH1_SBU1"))
 (segment (start 46.45 38.725) (end 46.45 38.3983) (width 0.2) (layer "F.Cu") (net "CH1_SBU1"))
 (segment (start 53.7992 41.3008) (end 54.45 41.9516) (width 0.2) (layer "F.Cu") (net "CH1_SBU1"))
 (segment (start 43.7717 47.3734) (end 44.3983 48) (width 0.2) (layer "F.Cu") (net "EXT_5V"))
 (segment (start 51.5519 47.0983) (end 53.0553 48.6017) (width 0.2) (layer "F.Cu") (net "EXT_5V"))
 (segment (start 37.2492 48) (end 36.9483 48) (width 0.2) (layer "F.Cu") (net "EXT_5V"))
 (segment (start 37.2492 48) (end 37.8758 47.3734) (width 0.2) (layer "F.Cu") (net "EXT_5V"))
 (segment (start 28.7293 48.219) (end 28.9483 48) (width 0.2) (layer "F.Cu") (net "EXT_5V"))
 (segment (start 29.55 48) (end 28.9483 48) (width 0.2) (layer "F.Cu") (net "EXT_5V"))
 (segment (start 53.0553 48.6017) (end 60.3466 48.6017) (width 0.2) (layer "F.Cu") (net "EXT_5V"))
 (segment (start 37.55 48) (end 37.2492 48) (width 0.2) (layer "F.Cu") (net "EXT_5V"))
 (segment (start 37.8758 47.3734) (end 43.7717 47.3734) (width 0.2) (layer "F.Cu") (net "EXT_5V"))
 (segment (start 29.112 48.6017) (end 36.3466 48.6017) (width 0.2) (layer "F.Cu") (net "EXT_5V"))
 (segment (start 45.1 48) (end 44.3983 48) (width 0.2) (layer "F.Cu") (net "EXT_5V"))
 (segment (start 61.55 48) (end 60.9483 48) (width 0.2) (layer "F.Cu") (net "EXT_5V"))
 (segment (start 28.7293 48.219) (end 29.112 48.6017) (width 0.2) (layer "F.Cu") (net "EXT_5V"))
 (segment (start 36.3466 48.6017) (end 36.9483 48) (width 0.2) (layer "F.Cu") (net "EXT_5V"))
 (segment (start 60.3466 48.6017) (end 60.9483 48) (width 0.2) (layer "F.Cu") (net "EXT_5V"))
 (segment (start 44.3983 48) (end 45.3 47.0983) (width 0.2) (layer "F.Cu") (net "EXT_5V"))
 (segment (start 45.3 47.0983) (end 51.5519 47.0983) (width 0.2) (layer "F.Cu") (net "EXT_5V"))
 (via (at 28.7293 48.219) (size 0.6) (drill 0.3) (layers "F.Cu" "B.Cu") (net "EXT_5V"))
 (segment (start 30 30) (end 30 46.9483) (width 0.2) (layer "B.Cu") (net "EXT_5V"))
 (segment (start 32.54 30) (end 30 30) (width 0.2) (layer "B.Cu") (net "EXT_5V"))
 (segment (start 30 30) (end 27.46 30) (width 0.2) (layer "B.Cu") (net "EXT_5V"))
 (segment (start 33.81 31.27) (end 32.54 30) (width 0.2) (layer "B.Cu") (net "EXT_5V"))
 (segment (start 27.46 30) (end 26.19 28.73) (width 0.2) (layer "B.Cu") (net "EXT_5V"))
 (segment (start 30 46.9483) (end 28.7293 48.219) (width 0.2) (layer "B.Cu") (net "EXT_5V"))
 (segment (start 37.05 27.7982) (end 36.623 27.7982) (width 0.2) (layer "F.Cu") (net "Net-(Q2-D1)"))
 (segment (start 37.55 38.1808) (end 37.55 39) (width 0.2) (layer "F.Cu") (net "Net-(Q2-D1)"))
 (segment (start 37.05 28.6999) (end 37.05 27.7982) (width 0.2) (layer "F.Cu") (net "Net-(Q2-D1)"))
 (segment (start 36.623 27.7982) (end 36.4824 27.6576) (width 0.2) (layer "F.Cu") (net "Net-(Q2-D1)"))
 (via (at 37.55 38.1808) (size 0.6) (drill 0.3) (layers "F.Cu" "B.Cu") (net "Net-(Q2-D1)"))
 (via (at 36.4824 27.6576) (size 0.6) (drill 0.3) (layers "F.Cu" "B.Cu") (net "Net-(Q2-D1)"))
 (segment (start 36.4824 37.1132) (end 37.55 38.1808) (width 0.2) (layer "B.Cu") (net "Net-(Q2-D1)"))
 (segment (start 36.4824 27.6576) (end 36.4824 37.1132) (width 0.2) (layer "B.Cu") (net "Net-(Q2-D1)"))
 (segment (start 51.0184 46.0666) (end 32.9851 46.0666) (width 0.2) (layer "F.Cu") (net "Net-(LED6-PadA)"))
 (segment (start 62 40.05) (end 57.035 40.05) (width 0.2) (layer "F.Cu") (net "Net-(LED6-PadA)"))
 (segment (start 32.9851 46.0666) (end 31.0517 48) (width 0.2) (layer "F.Cu") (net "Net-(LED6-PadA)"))
 (segment (start 30.45 48) (end 31.0517 48) (width 0.2) (layer "F.Cu") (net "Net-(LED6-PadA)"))
 (via (at 51.0184 46.0666) (size 0.6) (drill 0.3) (layers "F.Cu" "B.Cu") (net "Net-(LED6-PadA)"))
 (via (at 57.035 40.05) (size 0.6) (drill 0.3) (layers "F.Cu" "B.Cu") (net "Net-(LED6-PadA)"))
 (segment (start 51.0184 46.0666) (end 57.035 40.05) (width 0.2) (layer "B.Cu") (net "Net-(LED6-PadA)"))
 (segment (start 37.05 31.3001) (end 37.05 32.2018) (width 0.2) (layer "F.Cu") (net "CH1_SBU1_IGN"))
 (segment (start 30.45 39) (end 30.45 32.99) (width 0.2) (layer "F.Cu") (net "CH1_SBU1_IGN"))
 (segment (start 29.9715 30.0285) (end 35.7784 30.0285) (width 0.2) (layer "F.Cu") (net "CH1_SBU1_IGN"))
 (segment (start 42.3448 32.6035) (end 44.9483 30) (width 0.2) (layer "F.Cu") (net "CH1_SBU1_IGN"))
 (segment (start 45.55 30) (end 44.9483 30) (width 0.2) (layer "F.Cu") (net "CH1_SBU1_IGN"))
 (segment (start 35.7784 30.0285) (end 37.05 31.3001) (width 0.2) (layer "F.Cu") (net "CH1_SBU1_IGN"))
 (segment (start 28.73 31.27) (end 29.9715 30.0285) (width 0.2) (layer "F.Cu") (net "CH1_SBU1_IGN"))
 (segment (start 37.4517 32.6035) (end 42.3448 32.6035) (width 0.2) (layer "F.Cu") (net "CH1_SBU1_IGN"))
 (segment (start 37.05 32.2018) (end 37.4517 32.6035) (width 0.2) (layer "F.Cu") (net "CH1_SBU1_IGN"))
 (segment (start 30.45 32.99) (end 28.73 31.27) (width 0.2) (layer "F.Cu") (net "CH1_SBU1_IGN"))
 (segment (start 29.55 39) (end 29.55 39.6017) (width 0.2) (layer "F.Cu") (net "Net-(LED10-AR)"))
 (segment (start 53.05 40) (end 52.3483 40) (width 0.2) (layer "F.Cu") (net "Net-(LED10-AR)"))
 (segment (start 51.8644 40.4839) (end 30.4322 40.4839) (width 0.2) (layer "F.Cu") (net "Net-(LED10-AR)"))
 (segment (start 30.4322 40.4839) (end 29.55 39.6017) (width 0.2) (layer "F.Cu") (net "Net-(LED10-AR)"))
 (segment (start 52.3483 40) (end 51.8644 40.4839) (width 0.2) (layer "F.Cu") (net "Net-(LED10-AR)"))
 (segment (start 54.95 40) (end 54.95 37.2017) (width 0.2) (layer "F.Cu") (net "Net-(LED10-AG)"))
 (segment (start 54.95 37.2017) (end 61.55 30.6017) (width 0.2) (layer "F.Cu") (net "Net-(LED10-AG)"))
 (segment (start 61.55 30) (end 61.55 30.6017) (width 0.2) (layer "F.Cu") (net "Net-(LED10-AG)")))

